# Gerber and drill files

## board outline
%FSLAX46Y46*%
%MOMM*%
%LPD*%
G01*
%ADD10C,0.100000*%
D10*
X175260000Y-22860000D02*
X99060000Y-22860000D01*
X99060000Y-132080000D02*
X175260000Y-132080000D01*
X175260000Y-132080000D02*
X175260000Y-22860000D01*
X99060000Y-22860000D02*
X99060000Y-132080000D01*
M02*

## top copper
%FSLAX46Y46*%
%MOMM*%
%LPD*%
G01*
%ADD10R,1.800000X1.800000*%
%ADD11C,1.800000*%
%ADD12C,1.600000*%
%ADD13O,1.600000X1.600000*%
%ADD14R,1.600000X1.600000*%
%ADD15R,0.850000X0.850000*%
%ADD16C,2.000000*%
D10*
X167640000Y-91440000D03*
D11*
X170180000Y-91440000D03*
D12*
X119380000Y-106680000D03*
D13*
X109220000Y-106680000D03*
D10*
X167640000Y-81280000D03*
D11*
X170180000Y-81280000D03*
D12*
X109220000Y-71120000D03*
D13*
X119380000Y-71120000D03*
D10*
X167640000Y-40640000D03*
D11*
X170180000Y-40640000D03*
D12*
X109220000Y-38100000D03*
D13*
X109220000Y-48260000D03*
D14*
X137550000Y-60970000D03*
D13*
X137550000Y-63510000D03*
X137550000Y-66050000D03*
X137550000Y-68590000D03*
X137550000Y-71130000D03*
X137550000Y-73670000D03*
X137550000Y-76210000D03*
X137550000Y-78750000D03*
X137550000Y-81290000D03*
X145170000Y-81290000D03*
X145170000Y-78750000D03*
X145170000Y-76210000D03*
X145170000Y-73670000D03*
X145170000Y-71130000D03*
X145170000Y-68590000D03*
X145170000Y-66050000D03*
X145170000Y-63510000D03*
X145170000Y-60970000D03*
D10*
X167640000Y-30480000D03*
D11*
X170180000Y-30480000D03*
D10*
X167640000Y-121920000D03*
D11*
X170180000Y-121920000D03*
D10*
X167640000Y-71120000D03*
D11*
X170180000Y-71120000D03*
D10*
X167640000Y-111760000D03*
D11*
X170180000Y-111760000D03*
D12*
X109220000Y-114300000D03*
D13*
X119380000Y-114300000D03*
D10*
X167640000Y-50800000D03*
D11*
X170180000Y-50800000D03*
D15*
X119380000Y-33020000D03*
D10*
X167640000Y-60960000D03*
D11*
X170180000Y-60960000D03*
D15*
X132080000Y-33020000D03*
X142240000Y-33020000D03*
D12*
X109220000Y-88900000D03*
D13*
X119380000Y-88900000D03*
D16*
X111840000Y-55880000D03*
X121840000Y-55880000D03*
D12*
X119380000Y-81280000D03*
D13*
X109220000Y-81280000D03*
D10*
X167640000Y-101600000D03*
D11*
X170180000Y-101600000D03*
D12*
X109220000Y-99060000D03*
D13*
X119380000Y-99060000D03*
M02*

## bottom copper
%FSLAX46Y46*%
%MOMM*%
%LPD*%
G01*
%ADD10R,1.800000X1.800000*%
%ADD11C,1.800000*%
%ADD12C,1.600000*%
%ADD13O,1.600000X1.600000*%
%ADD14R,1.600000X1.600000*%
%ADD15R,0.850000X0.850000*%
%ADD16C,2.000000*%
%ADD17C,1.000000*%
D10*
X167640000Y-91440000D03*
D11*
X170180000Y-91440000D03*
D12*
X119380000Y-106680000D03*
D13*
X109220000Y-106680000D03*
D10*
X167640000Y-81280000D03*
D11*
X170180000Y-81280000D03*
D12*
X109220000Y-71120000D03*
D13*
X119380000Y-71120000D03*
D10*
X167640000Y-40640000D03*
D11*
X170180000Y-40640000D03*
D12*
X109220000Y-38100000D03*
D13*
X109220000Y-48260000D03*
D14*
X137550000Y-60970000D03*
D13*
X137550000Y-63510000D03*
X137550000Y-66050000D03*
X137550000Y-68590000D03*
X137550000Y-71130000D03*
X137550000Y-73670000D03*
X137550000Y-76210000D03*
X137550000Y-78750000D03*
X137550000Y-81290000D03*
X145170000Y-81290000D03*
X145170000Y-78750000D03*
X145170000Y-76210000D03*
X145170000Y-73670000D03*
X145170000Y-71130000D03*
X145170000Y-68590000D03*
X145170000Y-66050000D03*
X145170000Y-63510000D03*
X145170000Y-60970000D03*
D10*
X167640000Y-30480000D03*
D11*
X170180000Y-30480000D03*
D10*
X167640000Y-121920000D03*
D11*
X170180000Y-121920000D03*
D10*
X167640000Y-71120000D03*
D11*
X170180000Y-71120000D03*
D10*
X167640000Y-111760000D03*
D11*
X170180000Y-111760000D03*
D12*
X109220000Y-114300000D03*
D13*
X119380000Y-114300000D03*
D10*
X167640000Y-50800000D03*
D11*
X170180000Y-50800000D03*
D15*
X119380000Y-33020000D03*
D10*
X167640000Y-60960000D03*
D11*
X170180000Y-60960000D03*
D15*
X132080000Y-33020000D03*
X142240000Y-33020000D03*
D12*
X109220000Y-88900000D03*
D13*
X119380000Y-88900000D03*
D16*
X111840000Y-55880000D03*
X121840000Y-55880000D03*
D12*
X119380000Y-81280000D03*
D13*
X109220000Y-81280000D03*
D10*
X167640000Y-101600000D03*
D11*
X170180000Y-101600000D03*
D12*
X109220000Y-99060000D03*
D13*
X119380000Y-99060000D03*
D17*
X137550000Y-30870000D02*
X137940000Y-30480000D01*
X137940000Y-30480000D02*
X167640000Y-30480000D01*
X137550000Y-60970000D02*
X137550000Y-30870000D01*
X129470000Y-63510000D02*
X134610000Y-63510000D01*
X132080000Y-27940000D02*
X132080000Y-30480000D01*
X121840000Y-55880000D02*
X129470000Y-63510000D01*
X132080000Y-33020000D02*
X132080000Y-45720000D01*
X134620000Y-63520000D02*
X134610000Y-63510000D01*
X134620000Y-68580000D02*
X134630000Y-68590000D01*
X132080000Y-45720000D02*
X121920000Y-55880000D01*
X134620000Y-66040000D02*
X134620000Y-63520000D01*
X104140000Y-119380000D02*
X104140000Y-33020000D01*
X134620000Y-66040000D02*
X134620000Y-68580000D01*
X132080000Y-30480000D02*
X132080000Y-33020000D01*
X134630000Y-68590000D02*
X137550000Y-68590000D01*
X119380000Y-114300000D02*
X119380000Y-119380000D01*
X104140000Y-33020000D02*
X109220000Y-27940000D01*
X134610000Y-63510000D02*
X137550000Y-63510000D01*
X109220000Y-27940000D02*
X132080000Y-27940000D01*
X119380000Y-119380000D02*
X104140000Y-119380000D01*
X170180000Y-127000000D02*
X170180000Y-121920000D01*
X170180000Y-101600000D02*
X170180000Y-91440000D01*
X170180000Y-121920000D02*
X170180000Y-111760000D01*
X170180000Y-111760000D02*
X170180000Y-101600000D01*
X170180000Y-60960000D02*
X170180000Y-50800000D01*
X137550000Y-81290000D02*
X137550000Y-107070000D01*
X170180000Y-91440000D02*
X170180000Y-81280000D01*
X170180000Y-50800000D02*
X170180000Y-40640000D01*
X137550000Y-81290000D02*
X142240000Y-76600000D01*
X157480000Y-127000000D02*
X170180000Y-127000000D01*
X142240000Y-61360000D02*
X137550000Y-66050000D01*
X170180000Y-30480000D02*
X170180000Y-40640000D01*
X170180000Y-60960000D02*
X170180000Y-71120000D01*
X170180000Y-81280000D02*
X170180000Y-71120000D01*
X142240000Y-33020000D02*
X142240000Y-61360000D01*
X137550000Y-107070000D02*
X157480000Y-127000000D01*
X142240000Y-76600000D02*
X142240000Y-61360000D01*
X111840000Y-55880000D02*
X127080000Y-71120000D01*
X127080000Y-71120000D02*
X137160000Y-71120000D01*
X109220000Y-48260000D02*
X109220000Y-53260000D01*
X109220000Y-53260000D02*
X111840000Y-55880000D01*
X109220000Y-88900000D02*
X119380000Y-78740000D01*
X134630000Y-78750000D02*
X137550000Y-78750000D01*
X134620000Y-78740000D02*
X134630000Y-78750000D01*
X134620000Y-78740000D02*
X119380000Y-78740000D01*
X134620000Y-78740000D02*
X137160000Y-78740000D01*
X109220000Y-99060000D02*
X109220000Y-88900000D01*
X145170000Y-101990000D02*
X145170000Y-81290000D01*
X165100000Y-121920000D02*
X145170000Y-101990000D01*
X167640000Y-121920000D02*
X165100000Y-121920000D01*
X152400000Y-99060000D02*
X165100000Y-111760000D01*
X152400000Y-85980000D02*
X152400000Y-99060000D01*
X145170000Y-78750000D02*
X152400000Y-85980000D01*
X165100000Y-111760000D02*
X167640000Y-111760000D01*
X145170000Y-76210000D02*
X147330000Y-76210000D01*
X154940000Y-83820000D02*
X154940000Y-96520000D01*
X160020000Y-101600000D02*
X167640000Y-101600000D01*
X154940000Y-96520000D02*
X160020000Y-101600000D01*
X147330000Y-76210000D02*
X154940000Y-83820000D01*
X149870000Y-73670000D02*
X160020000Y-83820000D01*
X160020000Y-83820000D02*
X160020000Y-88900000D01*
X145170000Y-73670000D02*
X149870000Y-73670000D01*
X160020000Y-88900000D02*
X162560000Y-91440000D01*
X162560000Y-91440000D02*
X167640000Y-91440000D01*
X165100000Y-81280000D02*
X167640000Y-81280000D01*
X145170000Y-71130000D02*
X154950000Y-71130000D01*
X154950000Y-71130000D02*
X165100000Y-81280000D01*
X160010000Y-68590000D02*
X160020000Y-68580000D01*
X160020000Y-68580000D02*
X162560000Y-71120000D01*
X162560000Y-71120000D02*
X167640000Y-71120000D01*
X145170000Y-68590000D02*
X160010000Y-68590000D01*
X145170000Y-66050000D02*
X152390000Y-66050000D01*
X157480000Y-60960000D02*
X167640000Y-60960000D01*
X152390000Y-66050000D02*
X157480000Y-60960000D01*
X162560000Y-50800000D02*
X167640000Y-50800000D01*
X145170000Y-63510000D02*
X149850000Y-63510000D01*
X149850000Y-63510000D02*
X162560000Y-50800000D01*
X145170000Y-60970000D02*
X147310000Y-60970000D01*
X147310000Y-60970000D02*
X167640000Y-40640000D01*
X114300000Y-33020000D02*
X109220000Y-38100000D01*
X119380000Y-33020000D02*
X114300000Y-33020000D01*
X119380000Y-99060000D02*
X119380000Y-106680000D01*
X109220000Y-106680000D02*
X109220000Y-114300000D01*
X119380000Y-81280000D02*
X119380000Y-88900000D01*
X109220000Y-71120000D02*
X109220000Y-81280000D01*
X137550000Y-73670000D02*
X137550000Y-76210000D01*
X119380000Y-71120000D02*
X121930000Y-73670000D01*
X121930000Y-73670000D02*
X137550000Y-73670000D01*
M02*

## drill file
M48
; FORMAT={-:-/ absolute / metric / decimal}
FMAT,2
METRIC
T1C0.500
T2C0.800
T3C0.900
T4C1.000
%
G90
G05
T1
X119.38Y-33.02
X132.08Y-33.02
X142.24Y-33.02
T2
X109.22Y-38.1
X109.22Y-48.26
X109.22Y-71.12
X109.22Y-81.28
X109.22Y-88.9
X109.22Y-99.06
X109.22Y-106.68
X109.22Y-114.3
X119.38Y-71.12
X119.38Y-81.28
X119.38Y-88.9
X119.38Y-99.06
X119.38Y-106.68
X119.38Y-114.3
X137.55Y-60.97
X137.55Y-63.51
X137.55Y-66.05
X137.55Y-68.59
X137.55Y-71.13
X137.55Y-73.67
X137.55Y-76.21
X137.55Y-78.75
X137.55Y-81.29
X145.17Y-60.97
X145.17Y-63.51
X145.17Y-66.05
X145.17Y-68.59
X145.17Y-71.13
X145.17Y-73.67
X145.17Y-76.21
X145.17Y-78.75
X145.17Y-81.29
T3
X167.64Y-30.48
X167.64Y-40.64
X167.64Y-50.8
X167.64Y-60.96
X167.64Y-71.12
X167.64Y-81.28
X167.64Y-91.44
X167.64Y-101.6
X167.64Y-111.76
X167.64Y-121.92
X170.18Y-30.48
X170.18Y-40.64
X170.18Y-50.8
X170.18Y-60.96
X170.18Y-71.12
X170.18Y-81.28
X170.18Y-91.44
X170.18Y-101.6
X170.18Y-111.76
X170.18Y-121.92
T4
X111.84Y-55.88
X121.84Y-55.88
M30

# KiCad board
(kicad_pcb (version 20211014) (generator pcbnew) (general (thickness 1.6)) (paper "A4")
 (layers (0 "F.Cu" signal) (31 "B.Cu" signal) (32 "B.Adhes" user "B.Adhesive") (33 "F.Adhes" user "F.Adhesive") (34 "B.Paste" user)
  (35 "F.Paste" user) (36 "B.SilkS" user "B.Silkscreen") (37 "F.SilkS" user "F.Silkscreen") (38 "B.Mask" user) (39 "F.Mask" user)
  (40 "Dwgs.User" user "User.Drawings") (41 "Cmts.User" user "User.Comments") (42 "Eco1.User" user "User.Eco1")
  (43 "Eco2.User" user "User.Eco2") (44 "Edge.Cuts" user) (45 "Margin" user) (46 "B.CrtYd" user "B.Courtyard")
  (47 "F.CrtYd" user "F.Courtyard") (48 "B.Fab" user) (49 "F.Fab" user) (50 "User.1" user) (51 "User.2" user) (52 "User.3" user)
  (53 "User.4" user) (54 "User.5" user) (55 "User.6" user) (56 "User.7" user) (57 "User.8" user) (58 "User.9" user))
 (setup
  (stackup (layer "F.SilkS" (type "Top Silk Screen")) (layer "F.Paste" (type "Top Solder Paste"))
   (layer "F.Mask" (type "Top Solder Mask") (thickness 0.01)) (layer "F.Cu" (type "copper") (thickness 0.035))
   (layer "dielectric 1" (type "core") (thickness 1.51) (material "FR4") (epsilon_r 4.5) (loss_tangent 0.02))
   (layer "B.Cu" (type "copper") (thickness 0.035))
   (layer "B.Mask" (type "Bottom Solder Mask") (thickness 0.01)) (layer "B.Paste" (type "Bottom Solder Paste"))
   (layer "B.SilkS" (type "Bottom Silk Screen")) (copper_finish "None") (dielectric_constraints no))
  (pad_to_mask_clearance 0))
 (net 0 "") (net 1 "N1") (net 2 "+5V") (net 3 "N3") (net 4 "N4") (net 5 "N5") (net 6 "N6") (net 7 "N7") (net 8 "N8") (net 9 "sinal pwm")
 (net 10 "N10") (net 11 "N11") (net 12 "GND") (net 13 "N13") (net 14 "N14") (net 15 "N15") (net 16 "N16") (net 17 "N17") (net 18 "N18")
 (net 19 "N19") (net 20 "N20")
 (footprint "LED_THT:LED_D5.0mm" (layer "F.Cu") (at 167.64 91.44)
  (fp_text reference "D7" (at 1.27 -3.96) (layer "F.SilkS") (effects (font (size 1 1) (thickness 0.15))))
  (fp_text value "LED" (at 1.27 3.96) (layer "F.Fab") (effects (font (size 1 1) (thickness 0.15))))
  (pad "1" thru_hole rect (at 0 0) (size 1.8 1.8) (drill 0.9) (layers *.Cu *.Mask) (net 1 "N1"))
  (pad "2" thru_hole circle (at 2.54 0) (size 1.8 1.8) (drill 0.9) (layers *.Cu *.Mask) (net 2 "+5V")))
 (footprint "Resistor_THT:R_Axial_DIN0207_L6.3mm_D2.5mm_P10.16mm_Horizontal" (layer "F.Cu") (at 119.38 106.68 180)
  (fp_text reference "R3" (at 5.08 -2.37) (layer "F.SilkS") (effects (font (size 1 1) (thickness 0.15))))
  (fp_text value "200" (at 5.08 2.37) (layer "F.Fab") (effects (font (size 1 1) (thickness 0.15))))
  (pad "1" thru_hole circle (at 0 0 180) (size 1.6 1.6) (drill 0.8) (layers *.Cu *.Mask) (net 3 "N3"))
  (pad "2" thru_hole oval (at 10.16 0 180) (size 1.6 1.6) (drill 0.8) (layers *.Cu *.Mask) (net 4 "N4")))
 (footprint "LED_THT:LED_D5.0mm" (layer "F.Cu") (at 167.64 81.28)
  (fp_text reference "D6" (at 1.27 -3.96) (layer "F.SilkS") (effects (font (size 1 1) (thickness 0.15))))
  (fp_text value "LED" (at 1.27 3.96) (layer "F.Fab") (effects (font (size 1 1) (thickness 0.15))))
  (pad "1" thru_hole rect (at 0 0) (size 1.8 1.8) (drill 0.9) (layers *.Cu *.Mask) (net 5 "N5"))
  (pad "2" thru_hole circle (at 2.54 0) (size 1.8 1.8) (drill 0.9) (layers *.Cu *.Mask) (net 2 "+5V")))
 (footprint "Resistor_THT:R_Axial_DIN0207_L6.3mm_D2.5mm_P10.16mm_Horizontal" (layer "F.Cu") (at 109.22 71.12)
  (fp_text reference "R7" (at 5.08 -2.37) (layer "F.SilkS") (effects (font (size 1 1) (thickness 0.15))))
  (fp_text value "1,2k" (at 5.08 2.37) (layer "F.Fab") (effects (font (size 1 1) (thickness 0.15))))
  (pad "1" thru_hole circle (at 0 0) (size 1.6 1.6) (drill 0.8) (layers *.Cu *.Mask) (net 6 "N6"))
  (pad "2" thru_hole oval (at 10.16 0) (size 1.6 1.6) (drill 0.8) (layers *.Cu *.Mask) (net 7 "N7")))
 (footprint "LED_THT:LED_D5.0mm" (layer "F.Cu") (at 167.64 40.64)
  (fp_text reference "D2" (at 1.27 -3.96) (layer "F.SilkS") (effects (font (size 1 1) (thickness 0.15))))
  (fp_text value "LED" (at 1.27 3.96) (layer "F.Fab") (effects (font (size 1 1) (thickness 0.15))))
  (pad "1" thru_hole rect (at 0 0) (size 1.8 1.8) (drill 0.9) (layers *.Cu *.Mask) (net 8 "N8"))
  (pad "2" thru_hole circle (at 2.54 0) (size 1.8 1.8) (drill 0.9) (layers *.Cu *.Mask) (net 2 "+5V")))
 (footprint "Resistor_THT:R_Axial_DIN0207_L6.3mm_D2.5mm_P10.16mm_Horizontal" (layer "F.Cu") (at 109.22 38.1 -90)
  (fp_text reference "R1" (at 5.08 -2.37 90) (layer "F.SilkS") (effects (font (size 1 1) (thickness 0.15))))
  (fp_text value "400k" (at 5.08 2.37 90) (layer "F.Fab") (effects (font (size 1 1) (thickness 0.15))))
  (pad "1" thru_hole circle (at 0 0 270) (size 1.6 1.6) (drill 0.8) (layers *.Cu *.Mask) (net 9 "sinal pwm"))
  (pad "2" thru_hole oval (at 10.16 0 270) (size 1.6 1.6) (drill 0.8) (layers *.Cu *.Mask) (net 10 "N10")))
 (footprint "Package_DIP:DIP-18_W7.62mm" (layer "F.Cu") (at 137.55 60.97)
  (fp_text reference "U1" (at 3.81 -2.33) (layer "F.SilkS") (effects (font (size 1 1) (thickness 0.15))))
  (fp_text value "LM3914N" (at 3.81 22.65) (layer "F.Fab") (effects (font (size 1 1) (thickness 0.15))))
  (pad "1" thru_hole rect (at 0 0) (size 1.6 1.6) (drill 0.8) (layers *.Cu *.Mask) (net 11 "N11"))
  (pad "2" thru_hole oval (at 0 2.54) (size 1.6 1.6) (drill 0.8) (layers *.Cu *.Mask) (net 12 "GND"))
  (pad "3" thru_hole oval (at 0 5.08) (size 1.6 1.6) (drill 0.8) (layers *.Cu *.Mask) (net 2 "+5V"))
  (pad "4" thru_hole oval (at 0 7.62) (size 1.6 1.6) (drill 0.8) (layers *.Cu *.Mask) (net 12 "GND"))
  (pad "5" thru_hole oval (at 0 10.16) (size 1.6 1.6) (drill 0.8) (layers *.Cu *.Mask) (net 10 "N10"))
  (pad "6" thru_hole oval (at 0 12.7) (size 1.6 1.6) (drill 0.8) (layers *.Cu *.Mask) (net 7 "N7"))
  (pad "7" thru_hole oval (at 0 15.24) (size 1.6 1.6) (drill 0.8) (layers *.Cu *.Mask) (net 7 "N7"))
  (pad "8" thru_hole oval (at 0 17.78) (size 1.6 1.6) (drill 0.8) (layers *.Cu *.Mask) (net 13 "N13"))
  (pad "9" thru_hole oval (at 0 20.32) (size 1.6 1.6) (drill 0.8) (layers *.Cu *.Mask) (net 2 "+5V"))
  (pad "10" thru_hole oval (at 7.62 20.32) (size 1.6 1.6) (drill 0.8) (layers *.Cu *.Mask) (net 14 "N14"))
  (pad "11" thru_hole oval (at 7.62 17.78) (size 1.6 1.6) (drill 0.8) (layers *.Cu *.Mask) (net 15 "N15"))
  (pad "12" thru_hole oval (at 7.62 15.24) (size 1.6 1.6) (drill 0.8) (layers *.Cu *.Mask) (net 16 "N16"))
  (pad "13" thru_hole oval (at 7.62 12.7) (size 1.6 1.6) (drill 0.8) (layers *.Cu *.Mask) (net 1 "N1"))
  (pad "14" thru_hole oval (at 7.62 10.16) (size 1.6 1.6) (drill 0.8) (layers *.Cu *.Mask) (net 5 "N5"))
  (pad "15" thru_hole oval (at 7.62 7.62) (size 1.6 1.6) (drill 0.8) (layers *.Cu *.Mask) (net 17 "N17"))
  (pad "16" thru_hole oval (at 7.62 5.08) (size 1.6 1.6) (drill 0.8) (layers *.Cu *.Mask) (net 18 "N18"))
  (pad "17" thru_hole oval (at 7.62 2.54) (size 1.6 1.6) (drill 0.8) (layers *.Cu *.Mask) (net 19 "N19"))
  (pad "18" thru_hole oval (at 7.62 0) (size 1.6 1.6) (drill 0.8) (layers *.Cu *.Mask) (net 8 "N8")))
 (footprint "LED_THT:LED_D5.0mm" (layer "F.Cu") (at 167.64 30.48)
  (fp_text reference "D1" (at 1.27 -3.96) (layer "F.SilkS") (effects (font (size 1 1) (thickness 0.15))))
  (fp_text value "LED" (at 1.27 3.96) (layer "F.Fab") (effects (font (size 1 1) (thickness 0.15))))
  (pad "1" thru_hole rect (at 0 0) (size 1.8 1.8) (drill 0.9) (layers *.Cu *.Mask) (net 11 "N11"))
  (pad "2" thru_hole circle (at 2.54 0) (size 1.8 1.8) (drill 0.9) (layers *.Cu *.Mask) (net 2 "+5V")))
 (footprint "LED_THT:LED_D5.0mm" (layer "F.Cu") (at 167.64 121.92)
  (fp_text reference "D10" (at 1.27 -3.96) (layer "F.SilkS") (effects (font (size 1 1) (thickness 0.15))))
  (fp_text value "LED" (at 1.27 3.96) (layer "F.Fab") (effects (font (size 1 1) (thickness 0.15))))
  (pad "1" thru_hole rect (at 0 0) (size 1.8 1.8) (drill 0.9) (layers *.Cu *.Mask) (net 14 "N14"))
  (pad "2" thru_hole circle (at 2.54 0) (size 1.8 1.8) (drill 0.9) (layers *.Cu *.Mask) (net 2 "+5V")))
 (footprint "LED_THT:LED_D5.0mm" (layer "F.Cu") (at 167.64 71.12)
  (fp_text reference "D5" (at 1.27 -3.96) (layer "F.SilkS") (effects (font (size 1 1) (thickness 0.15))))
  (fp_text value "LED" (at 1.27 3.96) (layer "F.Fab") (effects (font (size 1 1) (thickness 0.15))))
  (pad "1" thru_hole rect (at 0 0) (size 1.8 1.8) (drill 0.9) (layers *.Cu *.Mask) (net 17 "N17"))
  (pad "2" thru_hole circle (at 2.54 0) (size 1.8 1.8) (drill 0.9) (layers *.Cu *.Mask) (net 2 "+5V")))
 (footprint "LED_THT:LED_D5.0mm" (layer "F.Cu") (at 167.64 111.76)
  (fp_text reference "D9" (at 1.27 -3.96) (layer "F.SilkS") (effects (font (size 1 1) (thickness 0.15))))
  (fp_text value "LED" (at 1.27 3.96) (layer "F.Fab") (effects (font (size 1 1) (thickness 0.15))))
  (pad "1" thru_hole rect (at 0 0) (size 1.8 1.8) (drill 0.9) (layers *.Cu *.Mask) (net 15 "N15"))
  (pad "2" thru_hole circle (at 2.54 0) (size 1.8 1.8) (drill 0.9) (layers *.Cu *.Mask) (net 2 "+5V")))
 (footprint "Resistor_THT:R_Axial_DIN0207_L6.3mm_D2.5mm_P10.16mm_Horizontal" (layer "F.Cu") (at 109.22 114.3)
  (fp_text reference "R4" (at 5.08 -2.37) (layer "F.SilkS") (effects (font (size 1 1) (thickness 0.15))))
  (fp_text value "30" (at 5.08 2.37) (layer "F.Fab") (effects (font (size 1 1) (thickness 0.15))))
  (pad "1" thru_hole circle (at 0 0) (size 1.6 1.6) (drill 0.8) (layers *.Cu *.Mask) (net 4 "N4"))
  (pad "2" thru_hole oval (at 10.16 0) (size 1.6 1.6) (drill 0.8) (layers *.Cu *.Mask) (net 12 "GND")))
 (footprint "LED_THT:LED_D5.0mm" (layer "F.Cu") (at 167.64 50.8)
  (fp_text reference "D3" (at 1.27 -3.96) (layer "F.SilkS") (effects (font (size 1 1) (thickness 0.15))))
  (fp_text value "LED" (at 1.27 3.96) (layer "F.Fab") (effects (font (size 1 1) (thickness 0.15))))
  (pad "1" thru_hole rect (at 0 0) (size 1.8 1.8) (drill 0.9) (layers *.Cu *.Mask) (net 19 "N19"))
  (pad "2" thru_hole circle (at 2.54 0) (size 1.8 1.8) (drill 0.9) (layers *.Cu *.Mask) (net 2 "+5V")))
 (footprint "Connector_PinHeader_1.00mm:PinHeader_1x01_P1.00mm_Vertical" (layer "F.Cu") (at 119.38 33.02)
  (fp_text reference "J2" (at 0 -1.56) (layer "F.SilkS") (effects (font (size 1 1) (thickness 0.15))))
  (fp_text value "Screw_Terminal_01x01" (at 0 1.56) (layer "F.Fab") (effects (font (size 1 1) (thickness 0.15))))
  (pad "1" thru_hole rect (at 0 0) (size 0.85 0.85) (drill 0.5) (layers *.Cu *.Mask) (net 9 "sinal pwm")))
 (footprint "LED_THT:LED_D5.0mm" (layer "F.Cu") (at 167.64 60.96)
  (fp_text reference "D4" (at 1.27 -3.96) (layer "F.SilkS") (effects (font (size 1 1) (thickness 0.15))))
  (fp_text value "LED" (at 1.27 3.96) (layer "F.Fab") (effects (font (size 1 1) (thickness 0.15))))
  (pad "1" thru_hole rect (at 0 0) (size 1.8 1.8) (drill 0.9) (layers *.Cu *.Mask) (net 18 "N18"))
  (pad "2" thru_hole circle (at 2.54 0) (size 1.8 1.8) (drill 0.9) (layers *.Cu *.Mask) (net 2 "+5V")))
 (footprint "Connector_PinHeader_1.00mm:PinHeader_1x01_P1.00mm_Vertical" (layer "F.Cu") (at 132.08 33.02)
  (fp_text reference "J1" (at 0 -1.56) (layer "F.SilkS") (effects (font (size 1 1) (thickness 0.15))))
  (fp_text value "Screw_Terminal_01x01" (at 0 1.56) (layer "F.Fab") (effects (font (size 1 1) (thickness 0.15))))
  (pad "1" thru_hole rect (at 0 0) (size 0.85 0.85) (drill 0.5) (layers *.Cu *.Mask) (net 12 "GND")))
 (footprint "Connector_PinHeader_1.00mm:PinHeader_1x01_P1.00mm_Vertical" (layer "F.Cu") (at 142.24 33.02)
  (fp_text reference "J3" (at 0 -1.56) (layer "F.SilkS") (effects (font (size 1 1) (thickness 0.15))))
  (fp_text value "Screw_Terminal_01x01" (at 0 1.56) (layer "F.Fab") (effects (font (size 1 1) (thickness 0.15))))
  (pad "1" thru_hole rect (at 0 0) (size 0.85 0.85) (drill 0.5) (layers *.Cu *.Mask) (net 2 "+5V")))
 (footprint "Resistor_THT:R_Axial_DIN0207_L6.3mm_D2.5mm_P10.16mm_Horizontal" (layer "F.Cu") (at 109.22 88.9)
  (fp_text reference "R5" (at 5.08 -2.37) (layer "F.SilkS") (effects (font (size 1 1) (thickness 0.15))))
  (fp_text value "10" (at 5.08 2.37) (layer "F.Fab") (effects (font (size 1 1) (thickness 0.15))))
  (pad "1" thru_hole circle (at 0 0) (size 1.6 1.6) (drill 0.8) (layers *.Cu *.Mask) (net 13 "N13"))
  (pad "2" thru_hole oval (at 10.16 0) (size 1.6 1.6) (drill 0.8) (layers *.Cu *.Mask) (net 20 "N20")))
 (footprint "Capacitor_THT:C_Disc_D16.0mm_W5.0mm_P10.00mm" (layer "F.Cu") (at 111.84 55.88)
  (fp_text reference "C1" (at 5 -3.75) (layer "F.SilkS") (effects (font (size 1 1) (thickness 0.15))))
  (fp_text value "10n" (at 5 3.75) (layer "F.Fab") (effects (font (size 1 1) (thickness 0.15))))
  (pad "1" thru_hole circle (at 0 0) (size 2 2) (drill 1) (layers *.Cu *.Mask) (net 10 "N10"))
  (pad "2" thru_hole circle (at 10 0) (size 2 2) (drill 1) (layers *.Cu *.Mask) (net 12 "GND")))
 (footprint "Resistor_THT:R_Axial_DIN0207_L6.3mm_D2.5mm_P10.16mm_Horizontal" (layer "F.Cu") (at 119.38 81.28 180)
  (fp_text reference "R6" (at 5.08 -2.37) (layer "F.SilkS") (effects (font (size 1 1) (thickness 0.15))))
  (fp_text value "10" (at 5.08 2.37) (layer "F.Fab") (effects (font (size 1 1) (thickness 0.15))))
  (pad "1" thru_hole circle (at 0 0 180) (size 1.6 1.6) (drill 0.8) (layers *.Cu *.Mask) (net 20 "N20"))
  (pad "2" thru_hole oval (at 10.16 0 180) (size 1.6 1.6) (drill 0.8) (layers *.Cu *.Mask) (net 6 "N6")))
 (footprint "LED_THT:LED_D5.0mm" (layer "F.Cu") (at 167.64 101.6)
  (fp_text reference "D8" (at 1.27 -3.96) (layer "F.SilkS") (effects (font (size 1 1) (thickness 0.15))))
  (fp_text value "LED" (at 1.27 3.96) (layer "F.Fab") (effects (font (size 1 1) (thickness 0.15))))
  (pad "1" thru_hole rect (at 0 0) (size 1.8 1.8) (drill 0.9) (layers *.Cu *.Mask) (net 16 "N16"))
  (pad "2" thru_hole circle (at 2.54 0) (size 1.8 1.8) (drill 0.9) (layers *.Cu *.Mask) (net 2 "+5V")))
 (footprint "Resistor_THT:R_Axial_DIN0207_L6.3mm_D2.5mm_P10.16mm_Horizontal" (layer "F.Cu") (at 109.22 99.06)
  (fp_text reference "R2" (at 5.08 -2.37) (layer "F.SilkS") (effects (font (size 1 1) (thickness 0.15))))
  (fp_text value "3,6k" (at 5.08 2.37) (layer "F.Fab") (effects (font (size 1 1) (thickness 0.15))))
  (pad "1" thru_hole circle (at 0 0) (size 1.6 1.6) (drill 0.8) (layers *.Cu *.Mask) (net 13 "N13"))
  (pad "2" thru_hole oval (at 10.16 0) (size 1.6 1.6) (drill 0.8) (layers *.Cu *.Mask) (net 3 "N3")))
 (gr_rect (start 177.8 134.62) (end 177.8 134.62) (layer "B.Cu") (width 0.2) (fill none))
 (gr_line (start 175.26 22.86) (end 99.06 22.86) (layer "Edge.Cuts") (width 0.1))
 (gr_line (start 99.06 132.08) (end 175.26 132.08) (layer "Edge.Cuts") (width 0.1))
 (gr_line (start 175.26 132.08) (end 175.26 22.86) (layer "Edge.Cuts") (width 0.1))
 (gr_line (start 99.06 22.86) (end 99.06 132.08) (layer "Edge.Cuts") (width 0.1))
 (segment (start 137.55 30.87) (end 137.94 30.48) (width 1) (layer "B.Cu") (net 11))
 (segment (start 137.94 30.48) (end 167.64 30.48) (width 1) (layer "B.Cu") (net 11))
 (segment (start 137.55 60.97) (end 137.55 30.87) (width 1) (layer "B.Cu") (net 11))
 (segment (start 129.47 63.51) (end 134.61 63.51) (width 1) (layer "B.Cu") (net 12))
 (segment (start 132.08 27.94) (end 132.08 30.48) (width 1) (layer "B.Cu") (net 12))
 (segment (start 121.84 55.88) (end 129.47 63.51) (width 1) (layer "B.Cu") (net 12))
 (segment (start 132.08 33.02) (end 132.08 45.72) (width 1) (layer "B.Cu") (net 12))
 (segment (start 134.62 63.52) (end 134.61 63.51) (width 1) (layer "B.Cu") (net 12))
 (segment (start 134.62 68.58) (end 134.63 68.59) (width 1) (layer "B.Cu") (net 12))
 (segment (start 132.08 45.72) (end 121.92 55.88) (width 1) (layer "B.Cu") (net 12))
 (segment (start 134.62 66.04) (end 134.62 63.52) (width 1) (layer "B.Cu") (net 12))
 (segment (start 104.14 119.38) (end 104.14 33.02) (width 1) (layer "B.Cu") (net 12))
 (segment (start 134.62 66.04) (end 134.62 68.58) (width 1) (layer "B.Cu") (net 12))
 (segment (start 132.08 30.48) (end 132.08 33.02) (width 1) (layer "B.Cu") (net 12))
 (segment (start 134.63 68.59) (end 137.55 68.59) (width 1) (layer "B.Cu") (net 12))
 (segment (start 119.38 114.3) (end 119.38 119.38) (width 1) (layer "B.Cu") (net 12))
 (segment (start 104.14 33.02) (end 109.22 27.94) (width 1) (layer "B.Cu") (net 12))
 (segment (start 134.61 63.51) (end 137.55 63.51) (width 1) (layer "B.Cu") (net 12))
 (segment (start 109.22 27.94) (end 132.08 27.94) (width 1) (layer "B.Cu") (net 12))
 (segment (start 119.38 119.38) (end 104.14 119.38) (width 1) (layer "B.Cu") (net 12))
 (segment (start 170.18 127) (end 170.18 121.92) (width 1) (layer "B.Cu") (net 2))
 (segment (start 170.18 101.6) (end 170.18 91.44) (width 1) (layer "B.Cu") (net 2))
 (segment (start 170.18 121.92) (end 170.18 111.76) (width 1) (layer "B.Cu") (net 2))
 (segment (start 170.18 111.76) (end 170.18 101.6) (width 1) (layer "B.Cu") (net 2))
 (segment (start 170.18 60.96) (end 170.18 50.8) (width 1) (layer "B.Cu") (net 2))
 (segment (start 137.55 81.29) (end 137.55 107.07) (width 1) (layer "B.Cu") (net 2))
 (segment (start 170.18 91.44) (end 170.18 81.28) (width 1) (layer "B.Cu") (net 2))
 (segment (start 170.18 50.8) (end 170.18 40.64) (width 1) (layer "B.Cu") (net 2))
 (segment (start 137.55 81.29) (end 142.24 76.6) (width 1) (layer "B.Cu") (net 2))
 (segment (start 157.48 127) (end 170.18 127) (width 1) (layer "B.Cu") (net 2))
 (segment (start 142.24 61.36) (end 137.55 66.05) (width 1) (layer "B.Cu") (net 2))
 (segment (start 170.18 30.48) (end 170.18 40.64) (width 1) (layer "B.Cu") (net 2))
 (segment (start 170.18 60.96) (end 170.18 71.12) (width 1) (layer "B.Cu") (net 2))
 (segment (start 170.18 81.28) (end 170.18 71.12) (width 1) (layer "B.Cu") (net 2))
 (segment (start 142.24 33.02) (end 142.24 61.36) (width 1) (layer "B.Cu") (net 2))
 (segment (start 137.55 107.07) (end 157.48 127) (width 1) (layer "B.Cu") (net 2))
 (segment (start 142.24 76.6) (end 142.24 61.36) (width 1) (layer "B.Cu") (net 2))
 (segment (start 111.84 55.88) (end 127.08 71.12) (width 1) (layer "B.Cu") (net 10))
 (segment (start 127.08 71.12) (end 137.16 71.12) (width 1) (layer "B.Cu") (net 10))
 (segment (start 109.22 48.26) (end 109.22 53.26) (width 1) (layer "B.Cu") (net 10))
 (segment (start 109.22 53.26) (end 111.84 55.88) (width 1) (layer "B.Cu") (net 10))
 (segment (start 109.22 88.9) (end 119.38 78.74) (width 1) (layer "B.Cu") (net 13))
 (segment (start 134.63 78.75) (end 137.55 78.75) (width 1) (layer "B.Cu") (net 13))
 (segment (start 134.62 78.74) (end 134.63 78.75) (width 1) (layer "B.Cu") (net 13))
 (segment (start 134.62 78.74) (end 119.38 78.74) (width 1) (layer "B.Cu") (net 13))
 (segment (start 134.62 78.74) (end 137.16 78.74) (width 1) (layer "B.Cu") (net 13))
 (segment (start 109.22 99.06) (end 109.22 88.9) (width 1) (layer "B.Cu") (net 13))
 (segment (start 145.17 101.99) (end 145.17 81.29) (width 1) (layer "B.Cu") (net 14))
 (segment (start 165.1 121.92) (end 145.17 101.99) (width 1) (layer "B.Cu") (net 14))
 (segment (start 167.64 121.92) (end 165.1 121.92) (width 1) (layer "B.Cu") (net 14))
 (segment (start 152.4 99.06) (end 165.1 111.76) (width 1) (layer "B.Cu") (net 15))
 (segment (start 152.4 85.98) (end 152.4 99.06) (width 1) (layer "B.Cu") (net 15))
 (segment (start 145.17 78.75) (end 152.4 85.98) (width 1) (layer "B.Cu") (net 15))
 (segment (start 165.1 111.76) (end 167.64 111.76) (width 1) (layer "B.Cu") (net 15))
 (segment (start 145.17 76.21) (end 147.33 76.21) (width 1) (layer "B.Cu") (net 16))
 (segment (start 154.94 83.82) (end 154.94 96.52) (width 1) (layer "B.Cu") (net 16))
 (segment (start 160.02 101.6) (end 167.64 101.6) (width 1) (layer "B.Cu") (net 16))
 (segment (start 154.94 96.52) (end 160.02 101.6) (width 1) (layer "B.Cu") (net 16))
 (segment (start 147.33 76.21) (end 154.94 83.82) (width 1) (layer "B.Cu") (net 16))
 (segment (start 149.87 73.67) (end 160.02 83.82) (width 1) (layer "B.Cu") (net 1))
 (segment (start 160.02 83.82) (end 160.02 88.9) (width 1) (layer "B.Cu") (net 1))
 (segment (start 145.17 73.67) (end 149.87 73.67) (width 1) (layer "B.Cu") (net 1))
 (segment (start 160.02 88.9) (end 162.56 91.44) (width 1) (layer "B.Cu") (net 1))
 (segment (start 162.56 91.44) (end 167.64 91.44) (width 1) (layer "B.Cu") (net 1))
 (segment (start 165.1 81.28) (end 167.64 81.28) (width 1) (layer "B.Cu") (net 5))
 (segment (start 145.17 71.13) (end 154.95 71.13) (width 1) (layer "B.Cu") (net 5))
 (segment (start 154.95 71.13) (end 165.1 81.28) (width 1) (layer "B.Cu") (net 5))
 (segment (start 160.01 68.59) (end 160.02 68.58) (width 1) (layer "B.Cu") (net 17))
 (segment (start 160.02 68.58) (end 162.56 71.12) (width 1) (layer "B.Cu") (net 17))
 (segment (start 162.56 71.12) (end 167.64 71.12) (width 1) (layer "B.Cu") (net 17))
 (segment (start 145.17 68.59) (end 160.01 68.59) (width 1) (layer "B.Cu") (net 17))
 (segment (start 145.17 66.05) (end 152.39 66.05) (width 1) (layer "B.Cu") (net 18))
 (segment (start 157.48 60.96) (end 167.64 60.96) (width 1) (layer "B.Cu") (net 18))
 (segment (start 152.39 66.05) (end 157.48 60.96) (width 1) (layer "B.Cu") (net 18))
 (segment (start 162.56 50.8) (end 167.64 50.8) (width 1) (layer "B.Cu") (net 19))
 (segment (start 145.17 63.51) (end 149.85 63.51) (width 1) (layer "B.Cu") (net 19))
 (segment (start 149.85 63.51) (end 162.56 50.8) (width 1) (layer "B.Cu") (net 19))
 (segment (start 145.17 60.97) (end 147.31 60.97) (width 1) (layer "B.Cu") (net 8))
 (segment (start 147.31 60.97) (end 167.64 40.64) (width 1) (layer "B.Cu") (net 8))
 (segment (start 114.3 33.02) (end 109.22 38.1) (width 1) (layer "B.Cu") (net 9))
 (segment (start 119.38 33.02) (end 114.3 33.02) (width 1) (layer "B.Cu") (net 9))
 (segment (start 119.38 99.06) (end 119.38 106.68) (width 1) (layer "B.Cu") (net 3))
 (segment (start 109.22 106.68) (end 109.22 114.3) (width 1) (layer "B.Cu") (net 4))
 (segment (start 119.38 81.28) (end 119.38 88.9) (width 1) (layer "B.Cu") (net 20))
 (segment (start 109.22 71.12) (end 109.22 81.28) (width 1) (layer "B.Cu") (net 6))
 (segment (start 137.55 73.67) (end 137.55 76.21) (width 1) (layer "B.Cu") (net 7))
 (segment (start 119.38 71.12) (end 121.93 73.67) (width 1) (layer "B.Cu") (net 7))
 (segment (start 121.93 73.67) (end 137.55 73.67) (width 1) (layer "B.Cu") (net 7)))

